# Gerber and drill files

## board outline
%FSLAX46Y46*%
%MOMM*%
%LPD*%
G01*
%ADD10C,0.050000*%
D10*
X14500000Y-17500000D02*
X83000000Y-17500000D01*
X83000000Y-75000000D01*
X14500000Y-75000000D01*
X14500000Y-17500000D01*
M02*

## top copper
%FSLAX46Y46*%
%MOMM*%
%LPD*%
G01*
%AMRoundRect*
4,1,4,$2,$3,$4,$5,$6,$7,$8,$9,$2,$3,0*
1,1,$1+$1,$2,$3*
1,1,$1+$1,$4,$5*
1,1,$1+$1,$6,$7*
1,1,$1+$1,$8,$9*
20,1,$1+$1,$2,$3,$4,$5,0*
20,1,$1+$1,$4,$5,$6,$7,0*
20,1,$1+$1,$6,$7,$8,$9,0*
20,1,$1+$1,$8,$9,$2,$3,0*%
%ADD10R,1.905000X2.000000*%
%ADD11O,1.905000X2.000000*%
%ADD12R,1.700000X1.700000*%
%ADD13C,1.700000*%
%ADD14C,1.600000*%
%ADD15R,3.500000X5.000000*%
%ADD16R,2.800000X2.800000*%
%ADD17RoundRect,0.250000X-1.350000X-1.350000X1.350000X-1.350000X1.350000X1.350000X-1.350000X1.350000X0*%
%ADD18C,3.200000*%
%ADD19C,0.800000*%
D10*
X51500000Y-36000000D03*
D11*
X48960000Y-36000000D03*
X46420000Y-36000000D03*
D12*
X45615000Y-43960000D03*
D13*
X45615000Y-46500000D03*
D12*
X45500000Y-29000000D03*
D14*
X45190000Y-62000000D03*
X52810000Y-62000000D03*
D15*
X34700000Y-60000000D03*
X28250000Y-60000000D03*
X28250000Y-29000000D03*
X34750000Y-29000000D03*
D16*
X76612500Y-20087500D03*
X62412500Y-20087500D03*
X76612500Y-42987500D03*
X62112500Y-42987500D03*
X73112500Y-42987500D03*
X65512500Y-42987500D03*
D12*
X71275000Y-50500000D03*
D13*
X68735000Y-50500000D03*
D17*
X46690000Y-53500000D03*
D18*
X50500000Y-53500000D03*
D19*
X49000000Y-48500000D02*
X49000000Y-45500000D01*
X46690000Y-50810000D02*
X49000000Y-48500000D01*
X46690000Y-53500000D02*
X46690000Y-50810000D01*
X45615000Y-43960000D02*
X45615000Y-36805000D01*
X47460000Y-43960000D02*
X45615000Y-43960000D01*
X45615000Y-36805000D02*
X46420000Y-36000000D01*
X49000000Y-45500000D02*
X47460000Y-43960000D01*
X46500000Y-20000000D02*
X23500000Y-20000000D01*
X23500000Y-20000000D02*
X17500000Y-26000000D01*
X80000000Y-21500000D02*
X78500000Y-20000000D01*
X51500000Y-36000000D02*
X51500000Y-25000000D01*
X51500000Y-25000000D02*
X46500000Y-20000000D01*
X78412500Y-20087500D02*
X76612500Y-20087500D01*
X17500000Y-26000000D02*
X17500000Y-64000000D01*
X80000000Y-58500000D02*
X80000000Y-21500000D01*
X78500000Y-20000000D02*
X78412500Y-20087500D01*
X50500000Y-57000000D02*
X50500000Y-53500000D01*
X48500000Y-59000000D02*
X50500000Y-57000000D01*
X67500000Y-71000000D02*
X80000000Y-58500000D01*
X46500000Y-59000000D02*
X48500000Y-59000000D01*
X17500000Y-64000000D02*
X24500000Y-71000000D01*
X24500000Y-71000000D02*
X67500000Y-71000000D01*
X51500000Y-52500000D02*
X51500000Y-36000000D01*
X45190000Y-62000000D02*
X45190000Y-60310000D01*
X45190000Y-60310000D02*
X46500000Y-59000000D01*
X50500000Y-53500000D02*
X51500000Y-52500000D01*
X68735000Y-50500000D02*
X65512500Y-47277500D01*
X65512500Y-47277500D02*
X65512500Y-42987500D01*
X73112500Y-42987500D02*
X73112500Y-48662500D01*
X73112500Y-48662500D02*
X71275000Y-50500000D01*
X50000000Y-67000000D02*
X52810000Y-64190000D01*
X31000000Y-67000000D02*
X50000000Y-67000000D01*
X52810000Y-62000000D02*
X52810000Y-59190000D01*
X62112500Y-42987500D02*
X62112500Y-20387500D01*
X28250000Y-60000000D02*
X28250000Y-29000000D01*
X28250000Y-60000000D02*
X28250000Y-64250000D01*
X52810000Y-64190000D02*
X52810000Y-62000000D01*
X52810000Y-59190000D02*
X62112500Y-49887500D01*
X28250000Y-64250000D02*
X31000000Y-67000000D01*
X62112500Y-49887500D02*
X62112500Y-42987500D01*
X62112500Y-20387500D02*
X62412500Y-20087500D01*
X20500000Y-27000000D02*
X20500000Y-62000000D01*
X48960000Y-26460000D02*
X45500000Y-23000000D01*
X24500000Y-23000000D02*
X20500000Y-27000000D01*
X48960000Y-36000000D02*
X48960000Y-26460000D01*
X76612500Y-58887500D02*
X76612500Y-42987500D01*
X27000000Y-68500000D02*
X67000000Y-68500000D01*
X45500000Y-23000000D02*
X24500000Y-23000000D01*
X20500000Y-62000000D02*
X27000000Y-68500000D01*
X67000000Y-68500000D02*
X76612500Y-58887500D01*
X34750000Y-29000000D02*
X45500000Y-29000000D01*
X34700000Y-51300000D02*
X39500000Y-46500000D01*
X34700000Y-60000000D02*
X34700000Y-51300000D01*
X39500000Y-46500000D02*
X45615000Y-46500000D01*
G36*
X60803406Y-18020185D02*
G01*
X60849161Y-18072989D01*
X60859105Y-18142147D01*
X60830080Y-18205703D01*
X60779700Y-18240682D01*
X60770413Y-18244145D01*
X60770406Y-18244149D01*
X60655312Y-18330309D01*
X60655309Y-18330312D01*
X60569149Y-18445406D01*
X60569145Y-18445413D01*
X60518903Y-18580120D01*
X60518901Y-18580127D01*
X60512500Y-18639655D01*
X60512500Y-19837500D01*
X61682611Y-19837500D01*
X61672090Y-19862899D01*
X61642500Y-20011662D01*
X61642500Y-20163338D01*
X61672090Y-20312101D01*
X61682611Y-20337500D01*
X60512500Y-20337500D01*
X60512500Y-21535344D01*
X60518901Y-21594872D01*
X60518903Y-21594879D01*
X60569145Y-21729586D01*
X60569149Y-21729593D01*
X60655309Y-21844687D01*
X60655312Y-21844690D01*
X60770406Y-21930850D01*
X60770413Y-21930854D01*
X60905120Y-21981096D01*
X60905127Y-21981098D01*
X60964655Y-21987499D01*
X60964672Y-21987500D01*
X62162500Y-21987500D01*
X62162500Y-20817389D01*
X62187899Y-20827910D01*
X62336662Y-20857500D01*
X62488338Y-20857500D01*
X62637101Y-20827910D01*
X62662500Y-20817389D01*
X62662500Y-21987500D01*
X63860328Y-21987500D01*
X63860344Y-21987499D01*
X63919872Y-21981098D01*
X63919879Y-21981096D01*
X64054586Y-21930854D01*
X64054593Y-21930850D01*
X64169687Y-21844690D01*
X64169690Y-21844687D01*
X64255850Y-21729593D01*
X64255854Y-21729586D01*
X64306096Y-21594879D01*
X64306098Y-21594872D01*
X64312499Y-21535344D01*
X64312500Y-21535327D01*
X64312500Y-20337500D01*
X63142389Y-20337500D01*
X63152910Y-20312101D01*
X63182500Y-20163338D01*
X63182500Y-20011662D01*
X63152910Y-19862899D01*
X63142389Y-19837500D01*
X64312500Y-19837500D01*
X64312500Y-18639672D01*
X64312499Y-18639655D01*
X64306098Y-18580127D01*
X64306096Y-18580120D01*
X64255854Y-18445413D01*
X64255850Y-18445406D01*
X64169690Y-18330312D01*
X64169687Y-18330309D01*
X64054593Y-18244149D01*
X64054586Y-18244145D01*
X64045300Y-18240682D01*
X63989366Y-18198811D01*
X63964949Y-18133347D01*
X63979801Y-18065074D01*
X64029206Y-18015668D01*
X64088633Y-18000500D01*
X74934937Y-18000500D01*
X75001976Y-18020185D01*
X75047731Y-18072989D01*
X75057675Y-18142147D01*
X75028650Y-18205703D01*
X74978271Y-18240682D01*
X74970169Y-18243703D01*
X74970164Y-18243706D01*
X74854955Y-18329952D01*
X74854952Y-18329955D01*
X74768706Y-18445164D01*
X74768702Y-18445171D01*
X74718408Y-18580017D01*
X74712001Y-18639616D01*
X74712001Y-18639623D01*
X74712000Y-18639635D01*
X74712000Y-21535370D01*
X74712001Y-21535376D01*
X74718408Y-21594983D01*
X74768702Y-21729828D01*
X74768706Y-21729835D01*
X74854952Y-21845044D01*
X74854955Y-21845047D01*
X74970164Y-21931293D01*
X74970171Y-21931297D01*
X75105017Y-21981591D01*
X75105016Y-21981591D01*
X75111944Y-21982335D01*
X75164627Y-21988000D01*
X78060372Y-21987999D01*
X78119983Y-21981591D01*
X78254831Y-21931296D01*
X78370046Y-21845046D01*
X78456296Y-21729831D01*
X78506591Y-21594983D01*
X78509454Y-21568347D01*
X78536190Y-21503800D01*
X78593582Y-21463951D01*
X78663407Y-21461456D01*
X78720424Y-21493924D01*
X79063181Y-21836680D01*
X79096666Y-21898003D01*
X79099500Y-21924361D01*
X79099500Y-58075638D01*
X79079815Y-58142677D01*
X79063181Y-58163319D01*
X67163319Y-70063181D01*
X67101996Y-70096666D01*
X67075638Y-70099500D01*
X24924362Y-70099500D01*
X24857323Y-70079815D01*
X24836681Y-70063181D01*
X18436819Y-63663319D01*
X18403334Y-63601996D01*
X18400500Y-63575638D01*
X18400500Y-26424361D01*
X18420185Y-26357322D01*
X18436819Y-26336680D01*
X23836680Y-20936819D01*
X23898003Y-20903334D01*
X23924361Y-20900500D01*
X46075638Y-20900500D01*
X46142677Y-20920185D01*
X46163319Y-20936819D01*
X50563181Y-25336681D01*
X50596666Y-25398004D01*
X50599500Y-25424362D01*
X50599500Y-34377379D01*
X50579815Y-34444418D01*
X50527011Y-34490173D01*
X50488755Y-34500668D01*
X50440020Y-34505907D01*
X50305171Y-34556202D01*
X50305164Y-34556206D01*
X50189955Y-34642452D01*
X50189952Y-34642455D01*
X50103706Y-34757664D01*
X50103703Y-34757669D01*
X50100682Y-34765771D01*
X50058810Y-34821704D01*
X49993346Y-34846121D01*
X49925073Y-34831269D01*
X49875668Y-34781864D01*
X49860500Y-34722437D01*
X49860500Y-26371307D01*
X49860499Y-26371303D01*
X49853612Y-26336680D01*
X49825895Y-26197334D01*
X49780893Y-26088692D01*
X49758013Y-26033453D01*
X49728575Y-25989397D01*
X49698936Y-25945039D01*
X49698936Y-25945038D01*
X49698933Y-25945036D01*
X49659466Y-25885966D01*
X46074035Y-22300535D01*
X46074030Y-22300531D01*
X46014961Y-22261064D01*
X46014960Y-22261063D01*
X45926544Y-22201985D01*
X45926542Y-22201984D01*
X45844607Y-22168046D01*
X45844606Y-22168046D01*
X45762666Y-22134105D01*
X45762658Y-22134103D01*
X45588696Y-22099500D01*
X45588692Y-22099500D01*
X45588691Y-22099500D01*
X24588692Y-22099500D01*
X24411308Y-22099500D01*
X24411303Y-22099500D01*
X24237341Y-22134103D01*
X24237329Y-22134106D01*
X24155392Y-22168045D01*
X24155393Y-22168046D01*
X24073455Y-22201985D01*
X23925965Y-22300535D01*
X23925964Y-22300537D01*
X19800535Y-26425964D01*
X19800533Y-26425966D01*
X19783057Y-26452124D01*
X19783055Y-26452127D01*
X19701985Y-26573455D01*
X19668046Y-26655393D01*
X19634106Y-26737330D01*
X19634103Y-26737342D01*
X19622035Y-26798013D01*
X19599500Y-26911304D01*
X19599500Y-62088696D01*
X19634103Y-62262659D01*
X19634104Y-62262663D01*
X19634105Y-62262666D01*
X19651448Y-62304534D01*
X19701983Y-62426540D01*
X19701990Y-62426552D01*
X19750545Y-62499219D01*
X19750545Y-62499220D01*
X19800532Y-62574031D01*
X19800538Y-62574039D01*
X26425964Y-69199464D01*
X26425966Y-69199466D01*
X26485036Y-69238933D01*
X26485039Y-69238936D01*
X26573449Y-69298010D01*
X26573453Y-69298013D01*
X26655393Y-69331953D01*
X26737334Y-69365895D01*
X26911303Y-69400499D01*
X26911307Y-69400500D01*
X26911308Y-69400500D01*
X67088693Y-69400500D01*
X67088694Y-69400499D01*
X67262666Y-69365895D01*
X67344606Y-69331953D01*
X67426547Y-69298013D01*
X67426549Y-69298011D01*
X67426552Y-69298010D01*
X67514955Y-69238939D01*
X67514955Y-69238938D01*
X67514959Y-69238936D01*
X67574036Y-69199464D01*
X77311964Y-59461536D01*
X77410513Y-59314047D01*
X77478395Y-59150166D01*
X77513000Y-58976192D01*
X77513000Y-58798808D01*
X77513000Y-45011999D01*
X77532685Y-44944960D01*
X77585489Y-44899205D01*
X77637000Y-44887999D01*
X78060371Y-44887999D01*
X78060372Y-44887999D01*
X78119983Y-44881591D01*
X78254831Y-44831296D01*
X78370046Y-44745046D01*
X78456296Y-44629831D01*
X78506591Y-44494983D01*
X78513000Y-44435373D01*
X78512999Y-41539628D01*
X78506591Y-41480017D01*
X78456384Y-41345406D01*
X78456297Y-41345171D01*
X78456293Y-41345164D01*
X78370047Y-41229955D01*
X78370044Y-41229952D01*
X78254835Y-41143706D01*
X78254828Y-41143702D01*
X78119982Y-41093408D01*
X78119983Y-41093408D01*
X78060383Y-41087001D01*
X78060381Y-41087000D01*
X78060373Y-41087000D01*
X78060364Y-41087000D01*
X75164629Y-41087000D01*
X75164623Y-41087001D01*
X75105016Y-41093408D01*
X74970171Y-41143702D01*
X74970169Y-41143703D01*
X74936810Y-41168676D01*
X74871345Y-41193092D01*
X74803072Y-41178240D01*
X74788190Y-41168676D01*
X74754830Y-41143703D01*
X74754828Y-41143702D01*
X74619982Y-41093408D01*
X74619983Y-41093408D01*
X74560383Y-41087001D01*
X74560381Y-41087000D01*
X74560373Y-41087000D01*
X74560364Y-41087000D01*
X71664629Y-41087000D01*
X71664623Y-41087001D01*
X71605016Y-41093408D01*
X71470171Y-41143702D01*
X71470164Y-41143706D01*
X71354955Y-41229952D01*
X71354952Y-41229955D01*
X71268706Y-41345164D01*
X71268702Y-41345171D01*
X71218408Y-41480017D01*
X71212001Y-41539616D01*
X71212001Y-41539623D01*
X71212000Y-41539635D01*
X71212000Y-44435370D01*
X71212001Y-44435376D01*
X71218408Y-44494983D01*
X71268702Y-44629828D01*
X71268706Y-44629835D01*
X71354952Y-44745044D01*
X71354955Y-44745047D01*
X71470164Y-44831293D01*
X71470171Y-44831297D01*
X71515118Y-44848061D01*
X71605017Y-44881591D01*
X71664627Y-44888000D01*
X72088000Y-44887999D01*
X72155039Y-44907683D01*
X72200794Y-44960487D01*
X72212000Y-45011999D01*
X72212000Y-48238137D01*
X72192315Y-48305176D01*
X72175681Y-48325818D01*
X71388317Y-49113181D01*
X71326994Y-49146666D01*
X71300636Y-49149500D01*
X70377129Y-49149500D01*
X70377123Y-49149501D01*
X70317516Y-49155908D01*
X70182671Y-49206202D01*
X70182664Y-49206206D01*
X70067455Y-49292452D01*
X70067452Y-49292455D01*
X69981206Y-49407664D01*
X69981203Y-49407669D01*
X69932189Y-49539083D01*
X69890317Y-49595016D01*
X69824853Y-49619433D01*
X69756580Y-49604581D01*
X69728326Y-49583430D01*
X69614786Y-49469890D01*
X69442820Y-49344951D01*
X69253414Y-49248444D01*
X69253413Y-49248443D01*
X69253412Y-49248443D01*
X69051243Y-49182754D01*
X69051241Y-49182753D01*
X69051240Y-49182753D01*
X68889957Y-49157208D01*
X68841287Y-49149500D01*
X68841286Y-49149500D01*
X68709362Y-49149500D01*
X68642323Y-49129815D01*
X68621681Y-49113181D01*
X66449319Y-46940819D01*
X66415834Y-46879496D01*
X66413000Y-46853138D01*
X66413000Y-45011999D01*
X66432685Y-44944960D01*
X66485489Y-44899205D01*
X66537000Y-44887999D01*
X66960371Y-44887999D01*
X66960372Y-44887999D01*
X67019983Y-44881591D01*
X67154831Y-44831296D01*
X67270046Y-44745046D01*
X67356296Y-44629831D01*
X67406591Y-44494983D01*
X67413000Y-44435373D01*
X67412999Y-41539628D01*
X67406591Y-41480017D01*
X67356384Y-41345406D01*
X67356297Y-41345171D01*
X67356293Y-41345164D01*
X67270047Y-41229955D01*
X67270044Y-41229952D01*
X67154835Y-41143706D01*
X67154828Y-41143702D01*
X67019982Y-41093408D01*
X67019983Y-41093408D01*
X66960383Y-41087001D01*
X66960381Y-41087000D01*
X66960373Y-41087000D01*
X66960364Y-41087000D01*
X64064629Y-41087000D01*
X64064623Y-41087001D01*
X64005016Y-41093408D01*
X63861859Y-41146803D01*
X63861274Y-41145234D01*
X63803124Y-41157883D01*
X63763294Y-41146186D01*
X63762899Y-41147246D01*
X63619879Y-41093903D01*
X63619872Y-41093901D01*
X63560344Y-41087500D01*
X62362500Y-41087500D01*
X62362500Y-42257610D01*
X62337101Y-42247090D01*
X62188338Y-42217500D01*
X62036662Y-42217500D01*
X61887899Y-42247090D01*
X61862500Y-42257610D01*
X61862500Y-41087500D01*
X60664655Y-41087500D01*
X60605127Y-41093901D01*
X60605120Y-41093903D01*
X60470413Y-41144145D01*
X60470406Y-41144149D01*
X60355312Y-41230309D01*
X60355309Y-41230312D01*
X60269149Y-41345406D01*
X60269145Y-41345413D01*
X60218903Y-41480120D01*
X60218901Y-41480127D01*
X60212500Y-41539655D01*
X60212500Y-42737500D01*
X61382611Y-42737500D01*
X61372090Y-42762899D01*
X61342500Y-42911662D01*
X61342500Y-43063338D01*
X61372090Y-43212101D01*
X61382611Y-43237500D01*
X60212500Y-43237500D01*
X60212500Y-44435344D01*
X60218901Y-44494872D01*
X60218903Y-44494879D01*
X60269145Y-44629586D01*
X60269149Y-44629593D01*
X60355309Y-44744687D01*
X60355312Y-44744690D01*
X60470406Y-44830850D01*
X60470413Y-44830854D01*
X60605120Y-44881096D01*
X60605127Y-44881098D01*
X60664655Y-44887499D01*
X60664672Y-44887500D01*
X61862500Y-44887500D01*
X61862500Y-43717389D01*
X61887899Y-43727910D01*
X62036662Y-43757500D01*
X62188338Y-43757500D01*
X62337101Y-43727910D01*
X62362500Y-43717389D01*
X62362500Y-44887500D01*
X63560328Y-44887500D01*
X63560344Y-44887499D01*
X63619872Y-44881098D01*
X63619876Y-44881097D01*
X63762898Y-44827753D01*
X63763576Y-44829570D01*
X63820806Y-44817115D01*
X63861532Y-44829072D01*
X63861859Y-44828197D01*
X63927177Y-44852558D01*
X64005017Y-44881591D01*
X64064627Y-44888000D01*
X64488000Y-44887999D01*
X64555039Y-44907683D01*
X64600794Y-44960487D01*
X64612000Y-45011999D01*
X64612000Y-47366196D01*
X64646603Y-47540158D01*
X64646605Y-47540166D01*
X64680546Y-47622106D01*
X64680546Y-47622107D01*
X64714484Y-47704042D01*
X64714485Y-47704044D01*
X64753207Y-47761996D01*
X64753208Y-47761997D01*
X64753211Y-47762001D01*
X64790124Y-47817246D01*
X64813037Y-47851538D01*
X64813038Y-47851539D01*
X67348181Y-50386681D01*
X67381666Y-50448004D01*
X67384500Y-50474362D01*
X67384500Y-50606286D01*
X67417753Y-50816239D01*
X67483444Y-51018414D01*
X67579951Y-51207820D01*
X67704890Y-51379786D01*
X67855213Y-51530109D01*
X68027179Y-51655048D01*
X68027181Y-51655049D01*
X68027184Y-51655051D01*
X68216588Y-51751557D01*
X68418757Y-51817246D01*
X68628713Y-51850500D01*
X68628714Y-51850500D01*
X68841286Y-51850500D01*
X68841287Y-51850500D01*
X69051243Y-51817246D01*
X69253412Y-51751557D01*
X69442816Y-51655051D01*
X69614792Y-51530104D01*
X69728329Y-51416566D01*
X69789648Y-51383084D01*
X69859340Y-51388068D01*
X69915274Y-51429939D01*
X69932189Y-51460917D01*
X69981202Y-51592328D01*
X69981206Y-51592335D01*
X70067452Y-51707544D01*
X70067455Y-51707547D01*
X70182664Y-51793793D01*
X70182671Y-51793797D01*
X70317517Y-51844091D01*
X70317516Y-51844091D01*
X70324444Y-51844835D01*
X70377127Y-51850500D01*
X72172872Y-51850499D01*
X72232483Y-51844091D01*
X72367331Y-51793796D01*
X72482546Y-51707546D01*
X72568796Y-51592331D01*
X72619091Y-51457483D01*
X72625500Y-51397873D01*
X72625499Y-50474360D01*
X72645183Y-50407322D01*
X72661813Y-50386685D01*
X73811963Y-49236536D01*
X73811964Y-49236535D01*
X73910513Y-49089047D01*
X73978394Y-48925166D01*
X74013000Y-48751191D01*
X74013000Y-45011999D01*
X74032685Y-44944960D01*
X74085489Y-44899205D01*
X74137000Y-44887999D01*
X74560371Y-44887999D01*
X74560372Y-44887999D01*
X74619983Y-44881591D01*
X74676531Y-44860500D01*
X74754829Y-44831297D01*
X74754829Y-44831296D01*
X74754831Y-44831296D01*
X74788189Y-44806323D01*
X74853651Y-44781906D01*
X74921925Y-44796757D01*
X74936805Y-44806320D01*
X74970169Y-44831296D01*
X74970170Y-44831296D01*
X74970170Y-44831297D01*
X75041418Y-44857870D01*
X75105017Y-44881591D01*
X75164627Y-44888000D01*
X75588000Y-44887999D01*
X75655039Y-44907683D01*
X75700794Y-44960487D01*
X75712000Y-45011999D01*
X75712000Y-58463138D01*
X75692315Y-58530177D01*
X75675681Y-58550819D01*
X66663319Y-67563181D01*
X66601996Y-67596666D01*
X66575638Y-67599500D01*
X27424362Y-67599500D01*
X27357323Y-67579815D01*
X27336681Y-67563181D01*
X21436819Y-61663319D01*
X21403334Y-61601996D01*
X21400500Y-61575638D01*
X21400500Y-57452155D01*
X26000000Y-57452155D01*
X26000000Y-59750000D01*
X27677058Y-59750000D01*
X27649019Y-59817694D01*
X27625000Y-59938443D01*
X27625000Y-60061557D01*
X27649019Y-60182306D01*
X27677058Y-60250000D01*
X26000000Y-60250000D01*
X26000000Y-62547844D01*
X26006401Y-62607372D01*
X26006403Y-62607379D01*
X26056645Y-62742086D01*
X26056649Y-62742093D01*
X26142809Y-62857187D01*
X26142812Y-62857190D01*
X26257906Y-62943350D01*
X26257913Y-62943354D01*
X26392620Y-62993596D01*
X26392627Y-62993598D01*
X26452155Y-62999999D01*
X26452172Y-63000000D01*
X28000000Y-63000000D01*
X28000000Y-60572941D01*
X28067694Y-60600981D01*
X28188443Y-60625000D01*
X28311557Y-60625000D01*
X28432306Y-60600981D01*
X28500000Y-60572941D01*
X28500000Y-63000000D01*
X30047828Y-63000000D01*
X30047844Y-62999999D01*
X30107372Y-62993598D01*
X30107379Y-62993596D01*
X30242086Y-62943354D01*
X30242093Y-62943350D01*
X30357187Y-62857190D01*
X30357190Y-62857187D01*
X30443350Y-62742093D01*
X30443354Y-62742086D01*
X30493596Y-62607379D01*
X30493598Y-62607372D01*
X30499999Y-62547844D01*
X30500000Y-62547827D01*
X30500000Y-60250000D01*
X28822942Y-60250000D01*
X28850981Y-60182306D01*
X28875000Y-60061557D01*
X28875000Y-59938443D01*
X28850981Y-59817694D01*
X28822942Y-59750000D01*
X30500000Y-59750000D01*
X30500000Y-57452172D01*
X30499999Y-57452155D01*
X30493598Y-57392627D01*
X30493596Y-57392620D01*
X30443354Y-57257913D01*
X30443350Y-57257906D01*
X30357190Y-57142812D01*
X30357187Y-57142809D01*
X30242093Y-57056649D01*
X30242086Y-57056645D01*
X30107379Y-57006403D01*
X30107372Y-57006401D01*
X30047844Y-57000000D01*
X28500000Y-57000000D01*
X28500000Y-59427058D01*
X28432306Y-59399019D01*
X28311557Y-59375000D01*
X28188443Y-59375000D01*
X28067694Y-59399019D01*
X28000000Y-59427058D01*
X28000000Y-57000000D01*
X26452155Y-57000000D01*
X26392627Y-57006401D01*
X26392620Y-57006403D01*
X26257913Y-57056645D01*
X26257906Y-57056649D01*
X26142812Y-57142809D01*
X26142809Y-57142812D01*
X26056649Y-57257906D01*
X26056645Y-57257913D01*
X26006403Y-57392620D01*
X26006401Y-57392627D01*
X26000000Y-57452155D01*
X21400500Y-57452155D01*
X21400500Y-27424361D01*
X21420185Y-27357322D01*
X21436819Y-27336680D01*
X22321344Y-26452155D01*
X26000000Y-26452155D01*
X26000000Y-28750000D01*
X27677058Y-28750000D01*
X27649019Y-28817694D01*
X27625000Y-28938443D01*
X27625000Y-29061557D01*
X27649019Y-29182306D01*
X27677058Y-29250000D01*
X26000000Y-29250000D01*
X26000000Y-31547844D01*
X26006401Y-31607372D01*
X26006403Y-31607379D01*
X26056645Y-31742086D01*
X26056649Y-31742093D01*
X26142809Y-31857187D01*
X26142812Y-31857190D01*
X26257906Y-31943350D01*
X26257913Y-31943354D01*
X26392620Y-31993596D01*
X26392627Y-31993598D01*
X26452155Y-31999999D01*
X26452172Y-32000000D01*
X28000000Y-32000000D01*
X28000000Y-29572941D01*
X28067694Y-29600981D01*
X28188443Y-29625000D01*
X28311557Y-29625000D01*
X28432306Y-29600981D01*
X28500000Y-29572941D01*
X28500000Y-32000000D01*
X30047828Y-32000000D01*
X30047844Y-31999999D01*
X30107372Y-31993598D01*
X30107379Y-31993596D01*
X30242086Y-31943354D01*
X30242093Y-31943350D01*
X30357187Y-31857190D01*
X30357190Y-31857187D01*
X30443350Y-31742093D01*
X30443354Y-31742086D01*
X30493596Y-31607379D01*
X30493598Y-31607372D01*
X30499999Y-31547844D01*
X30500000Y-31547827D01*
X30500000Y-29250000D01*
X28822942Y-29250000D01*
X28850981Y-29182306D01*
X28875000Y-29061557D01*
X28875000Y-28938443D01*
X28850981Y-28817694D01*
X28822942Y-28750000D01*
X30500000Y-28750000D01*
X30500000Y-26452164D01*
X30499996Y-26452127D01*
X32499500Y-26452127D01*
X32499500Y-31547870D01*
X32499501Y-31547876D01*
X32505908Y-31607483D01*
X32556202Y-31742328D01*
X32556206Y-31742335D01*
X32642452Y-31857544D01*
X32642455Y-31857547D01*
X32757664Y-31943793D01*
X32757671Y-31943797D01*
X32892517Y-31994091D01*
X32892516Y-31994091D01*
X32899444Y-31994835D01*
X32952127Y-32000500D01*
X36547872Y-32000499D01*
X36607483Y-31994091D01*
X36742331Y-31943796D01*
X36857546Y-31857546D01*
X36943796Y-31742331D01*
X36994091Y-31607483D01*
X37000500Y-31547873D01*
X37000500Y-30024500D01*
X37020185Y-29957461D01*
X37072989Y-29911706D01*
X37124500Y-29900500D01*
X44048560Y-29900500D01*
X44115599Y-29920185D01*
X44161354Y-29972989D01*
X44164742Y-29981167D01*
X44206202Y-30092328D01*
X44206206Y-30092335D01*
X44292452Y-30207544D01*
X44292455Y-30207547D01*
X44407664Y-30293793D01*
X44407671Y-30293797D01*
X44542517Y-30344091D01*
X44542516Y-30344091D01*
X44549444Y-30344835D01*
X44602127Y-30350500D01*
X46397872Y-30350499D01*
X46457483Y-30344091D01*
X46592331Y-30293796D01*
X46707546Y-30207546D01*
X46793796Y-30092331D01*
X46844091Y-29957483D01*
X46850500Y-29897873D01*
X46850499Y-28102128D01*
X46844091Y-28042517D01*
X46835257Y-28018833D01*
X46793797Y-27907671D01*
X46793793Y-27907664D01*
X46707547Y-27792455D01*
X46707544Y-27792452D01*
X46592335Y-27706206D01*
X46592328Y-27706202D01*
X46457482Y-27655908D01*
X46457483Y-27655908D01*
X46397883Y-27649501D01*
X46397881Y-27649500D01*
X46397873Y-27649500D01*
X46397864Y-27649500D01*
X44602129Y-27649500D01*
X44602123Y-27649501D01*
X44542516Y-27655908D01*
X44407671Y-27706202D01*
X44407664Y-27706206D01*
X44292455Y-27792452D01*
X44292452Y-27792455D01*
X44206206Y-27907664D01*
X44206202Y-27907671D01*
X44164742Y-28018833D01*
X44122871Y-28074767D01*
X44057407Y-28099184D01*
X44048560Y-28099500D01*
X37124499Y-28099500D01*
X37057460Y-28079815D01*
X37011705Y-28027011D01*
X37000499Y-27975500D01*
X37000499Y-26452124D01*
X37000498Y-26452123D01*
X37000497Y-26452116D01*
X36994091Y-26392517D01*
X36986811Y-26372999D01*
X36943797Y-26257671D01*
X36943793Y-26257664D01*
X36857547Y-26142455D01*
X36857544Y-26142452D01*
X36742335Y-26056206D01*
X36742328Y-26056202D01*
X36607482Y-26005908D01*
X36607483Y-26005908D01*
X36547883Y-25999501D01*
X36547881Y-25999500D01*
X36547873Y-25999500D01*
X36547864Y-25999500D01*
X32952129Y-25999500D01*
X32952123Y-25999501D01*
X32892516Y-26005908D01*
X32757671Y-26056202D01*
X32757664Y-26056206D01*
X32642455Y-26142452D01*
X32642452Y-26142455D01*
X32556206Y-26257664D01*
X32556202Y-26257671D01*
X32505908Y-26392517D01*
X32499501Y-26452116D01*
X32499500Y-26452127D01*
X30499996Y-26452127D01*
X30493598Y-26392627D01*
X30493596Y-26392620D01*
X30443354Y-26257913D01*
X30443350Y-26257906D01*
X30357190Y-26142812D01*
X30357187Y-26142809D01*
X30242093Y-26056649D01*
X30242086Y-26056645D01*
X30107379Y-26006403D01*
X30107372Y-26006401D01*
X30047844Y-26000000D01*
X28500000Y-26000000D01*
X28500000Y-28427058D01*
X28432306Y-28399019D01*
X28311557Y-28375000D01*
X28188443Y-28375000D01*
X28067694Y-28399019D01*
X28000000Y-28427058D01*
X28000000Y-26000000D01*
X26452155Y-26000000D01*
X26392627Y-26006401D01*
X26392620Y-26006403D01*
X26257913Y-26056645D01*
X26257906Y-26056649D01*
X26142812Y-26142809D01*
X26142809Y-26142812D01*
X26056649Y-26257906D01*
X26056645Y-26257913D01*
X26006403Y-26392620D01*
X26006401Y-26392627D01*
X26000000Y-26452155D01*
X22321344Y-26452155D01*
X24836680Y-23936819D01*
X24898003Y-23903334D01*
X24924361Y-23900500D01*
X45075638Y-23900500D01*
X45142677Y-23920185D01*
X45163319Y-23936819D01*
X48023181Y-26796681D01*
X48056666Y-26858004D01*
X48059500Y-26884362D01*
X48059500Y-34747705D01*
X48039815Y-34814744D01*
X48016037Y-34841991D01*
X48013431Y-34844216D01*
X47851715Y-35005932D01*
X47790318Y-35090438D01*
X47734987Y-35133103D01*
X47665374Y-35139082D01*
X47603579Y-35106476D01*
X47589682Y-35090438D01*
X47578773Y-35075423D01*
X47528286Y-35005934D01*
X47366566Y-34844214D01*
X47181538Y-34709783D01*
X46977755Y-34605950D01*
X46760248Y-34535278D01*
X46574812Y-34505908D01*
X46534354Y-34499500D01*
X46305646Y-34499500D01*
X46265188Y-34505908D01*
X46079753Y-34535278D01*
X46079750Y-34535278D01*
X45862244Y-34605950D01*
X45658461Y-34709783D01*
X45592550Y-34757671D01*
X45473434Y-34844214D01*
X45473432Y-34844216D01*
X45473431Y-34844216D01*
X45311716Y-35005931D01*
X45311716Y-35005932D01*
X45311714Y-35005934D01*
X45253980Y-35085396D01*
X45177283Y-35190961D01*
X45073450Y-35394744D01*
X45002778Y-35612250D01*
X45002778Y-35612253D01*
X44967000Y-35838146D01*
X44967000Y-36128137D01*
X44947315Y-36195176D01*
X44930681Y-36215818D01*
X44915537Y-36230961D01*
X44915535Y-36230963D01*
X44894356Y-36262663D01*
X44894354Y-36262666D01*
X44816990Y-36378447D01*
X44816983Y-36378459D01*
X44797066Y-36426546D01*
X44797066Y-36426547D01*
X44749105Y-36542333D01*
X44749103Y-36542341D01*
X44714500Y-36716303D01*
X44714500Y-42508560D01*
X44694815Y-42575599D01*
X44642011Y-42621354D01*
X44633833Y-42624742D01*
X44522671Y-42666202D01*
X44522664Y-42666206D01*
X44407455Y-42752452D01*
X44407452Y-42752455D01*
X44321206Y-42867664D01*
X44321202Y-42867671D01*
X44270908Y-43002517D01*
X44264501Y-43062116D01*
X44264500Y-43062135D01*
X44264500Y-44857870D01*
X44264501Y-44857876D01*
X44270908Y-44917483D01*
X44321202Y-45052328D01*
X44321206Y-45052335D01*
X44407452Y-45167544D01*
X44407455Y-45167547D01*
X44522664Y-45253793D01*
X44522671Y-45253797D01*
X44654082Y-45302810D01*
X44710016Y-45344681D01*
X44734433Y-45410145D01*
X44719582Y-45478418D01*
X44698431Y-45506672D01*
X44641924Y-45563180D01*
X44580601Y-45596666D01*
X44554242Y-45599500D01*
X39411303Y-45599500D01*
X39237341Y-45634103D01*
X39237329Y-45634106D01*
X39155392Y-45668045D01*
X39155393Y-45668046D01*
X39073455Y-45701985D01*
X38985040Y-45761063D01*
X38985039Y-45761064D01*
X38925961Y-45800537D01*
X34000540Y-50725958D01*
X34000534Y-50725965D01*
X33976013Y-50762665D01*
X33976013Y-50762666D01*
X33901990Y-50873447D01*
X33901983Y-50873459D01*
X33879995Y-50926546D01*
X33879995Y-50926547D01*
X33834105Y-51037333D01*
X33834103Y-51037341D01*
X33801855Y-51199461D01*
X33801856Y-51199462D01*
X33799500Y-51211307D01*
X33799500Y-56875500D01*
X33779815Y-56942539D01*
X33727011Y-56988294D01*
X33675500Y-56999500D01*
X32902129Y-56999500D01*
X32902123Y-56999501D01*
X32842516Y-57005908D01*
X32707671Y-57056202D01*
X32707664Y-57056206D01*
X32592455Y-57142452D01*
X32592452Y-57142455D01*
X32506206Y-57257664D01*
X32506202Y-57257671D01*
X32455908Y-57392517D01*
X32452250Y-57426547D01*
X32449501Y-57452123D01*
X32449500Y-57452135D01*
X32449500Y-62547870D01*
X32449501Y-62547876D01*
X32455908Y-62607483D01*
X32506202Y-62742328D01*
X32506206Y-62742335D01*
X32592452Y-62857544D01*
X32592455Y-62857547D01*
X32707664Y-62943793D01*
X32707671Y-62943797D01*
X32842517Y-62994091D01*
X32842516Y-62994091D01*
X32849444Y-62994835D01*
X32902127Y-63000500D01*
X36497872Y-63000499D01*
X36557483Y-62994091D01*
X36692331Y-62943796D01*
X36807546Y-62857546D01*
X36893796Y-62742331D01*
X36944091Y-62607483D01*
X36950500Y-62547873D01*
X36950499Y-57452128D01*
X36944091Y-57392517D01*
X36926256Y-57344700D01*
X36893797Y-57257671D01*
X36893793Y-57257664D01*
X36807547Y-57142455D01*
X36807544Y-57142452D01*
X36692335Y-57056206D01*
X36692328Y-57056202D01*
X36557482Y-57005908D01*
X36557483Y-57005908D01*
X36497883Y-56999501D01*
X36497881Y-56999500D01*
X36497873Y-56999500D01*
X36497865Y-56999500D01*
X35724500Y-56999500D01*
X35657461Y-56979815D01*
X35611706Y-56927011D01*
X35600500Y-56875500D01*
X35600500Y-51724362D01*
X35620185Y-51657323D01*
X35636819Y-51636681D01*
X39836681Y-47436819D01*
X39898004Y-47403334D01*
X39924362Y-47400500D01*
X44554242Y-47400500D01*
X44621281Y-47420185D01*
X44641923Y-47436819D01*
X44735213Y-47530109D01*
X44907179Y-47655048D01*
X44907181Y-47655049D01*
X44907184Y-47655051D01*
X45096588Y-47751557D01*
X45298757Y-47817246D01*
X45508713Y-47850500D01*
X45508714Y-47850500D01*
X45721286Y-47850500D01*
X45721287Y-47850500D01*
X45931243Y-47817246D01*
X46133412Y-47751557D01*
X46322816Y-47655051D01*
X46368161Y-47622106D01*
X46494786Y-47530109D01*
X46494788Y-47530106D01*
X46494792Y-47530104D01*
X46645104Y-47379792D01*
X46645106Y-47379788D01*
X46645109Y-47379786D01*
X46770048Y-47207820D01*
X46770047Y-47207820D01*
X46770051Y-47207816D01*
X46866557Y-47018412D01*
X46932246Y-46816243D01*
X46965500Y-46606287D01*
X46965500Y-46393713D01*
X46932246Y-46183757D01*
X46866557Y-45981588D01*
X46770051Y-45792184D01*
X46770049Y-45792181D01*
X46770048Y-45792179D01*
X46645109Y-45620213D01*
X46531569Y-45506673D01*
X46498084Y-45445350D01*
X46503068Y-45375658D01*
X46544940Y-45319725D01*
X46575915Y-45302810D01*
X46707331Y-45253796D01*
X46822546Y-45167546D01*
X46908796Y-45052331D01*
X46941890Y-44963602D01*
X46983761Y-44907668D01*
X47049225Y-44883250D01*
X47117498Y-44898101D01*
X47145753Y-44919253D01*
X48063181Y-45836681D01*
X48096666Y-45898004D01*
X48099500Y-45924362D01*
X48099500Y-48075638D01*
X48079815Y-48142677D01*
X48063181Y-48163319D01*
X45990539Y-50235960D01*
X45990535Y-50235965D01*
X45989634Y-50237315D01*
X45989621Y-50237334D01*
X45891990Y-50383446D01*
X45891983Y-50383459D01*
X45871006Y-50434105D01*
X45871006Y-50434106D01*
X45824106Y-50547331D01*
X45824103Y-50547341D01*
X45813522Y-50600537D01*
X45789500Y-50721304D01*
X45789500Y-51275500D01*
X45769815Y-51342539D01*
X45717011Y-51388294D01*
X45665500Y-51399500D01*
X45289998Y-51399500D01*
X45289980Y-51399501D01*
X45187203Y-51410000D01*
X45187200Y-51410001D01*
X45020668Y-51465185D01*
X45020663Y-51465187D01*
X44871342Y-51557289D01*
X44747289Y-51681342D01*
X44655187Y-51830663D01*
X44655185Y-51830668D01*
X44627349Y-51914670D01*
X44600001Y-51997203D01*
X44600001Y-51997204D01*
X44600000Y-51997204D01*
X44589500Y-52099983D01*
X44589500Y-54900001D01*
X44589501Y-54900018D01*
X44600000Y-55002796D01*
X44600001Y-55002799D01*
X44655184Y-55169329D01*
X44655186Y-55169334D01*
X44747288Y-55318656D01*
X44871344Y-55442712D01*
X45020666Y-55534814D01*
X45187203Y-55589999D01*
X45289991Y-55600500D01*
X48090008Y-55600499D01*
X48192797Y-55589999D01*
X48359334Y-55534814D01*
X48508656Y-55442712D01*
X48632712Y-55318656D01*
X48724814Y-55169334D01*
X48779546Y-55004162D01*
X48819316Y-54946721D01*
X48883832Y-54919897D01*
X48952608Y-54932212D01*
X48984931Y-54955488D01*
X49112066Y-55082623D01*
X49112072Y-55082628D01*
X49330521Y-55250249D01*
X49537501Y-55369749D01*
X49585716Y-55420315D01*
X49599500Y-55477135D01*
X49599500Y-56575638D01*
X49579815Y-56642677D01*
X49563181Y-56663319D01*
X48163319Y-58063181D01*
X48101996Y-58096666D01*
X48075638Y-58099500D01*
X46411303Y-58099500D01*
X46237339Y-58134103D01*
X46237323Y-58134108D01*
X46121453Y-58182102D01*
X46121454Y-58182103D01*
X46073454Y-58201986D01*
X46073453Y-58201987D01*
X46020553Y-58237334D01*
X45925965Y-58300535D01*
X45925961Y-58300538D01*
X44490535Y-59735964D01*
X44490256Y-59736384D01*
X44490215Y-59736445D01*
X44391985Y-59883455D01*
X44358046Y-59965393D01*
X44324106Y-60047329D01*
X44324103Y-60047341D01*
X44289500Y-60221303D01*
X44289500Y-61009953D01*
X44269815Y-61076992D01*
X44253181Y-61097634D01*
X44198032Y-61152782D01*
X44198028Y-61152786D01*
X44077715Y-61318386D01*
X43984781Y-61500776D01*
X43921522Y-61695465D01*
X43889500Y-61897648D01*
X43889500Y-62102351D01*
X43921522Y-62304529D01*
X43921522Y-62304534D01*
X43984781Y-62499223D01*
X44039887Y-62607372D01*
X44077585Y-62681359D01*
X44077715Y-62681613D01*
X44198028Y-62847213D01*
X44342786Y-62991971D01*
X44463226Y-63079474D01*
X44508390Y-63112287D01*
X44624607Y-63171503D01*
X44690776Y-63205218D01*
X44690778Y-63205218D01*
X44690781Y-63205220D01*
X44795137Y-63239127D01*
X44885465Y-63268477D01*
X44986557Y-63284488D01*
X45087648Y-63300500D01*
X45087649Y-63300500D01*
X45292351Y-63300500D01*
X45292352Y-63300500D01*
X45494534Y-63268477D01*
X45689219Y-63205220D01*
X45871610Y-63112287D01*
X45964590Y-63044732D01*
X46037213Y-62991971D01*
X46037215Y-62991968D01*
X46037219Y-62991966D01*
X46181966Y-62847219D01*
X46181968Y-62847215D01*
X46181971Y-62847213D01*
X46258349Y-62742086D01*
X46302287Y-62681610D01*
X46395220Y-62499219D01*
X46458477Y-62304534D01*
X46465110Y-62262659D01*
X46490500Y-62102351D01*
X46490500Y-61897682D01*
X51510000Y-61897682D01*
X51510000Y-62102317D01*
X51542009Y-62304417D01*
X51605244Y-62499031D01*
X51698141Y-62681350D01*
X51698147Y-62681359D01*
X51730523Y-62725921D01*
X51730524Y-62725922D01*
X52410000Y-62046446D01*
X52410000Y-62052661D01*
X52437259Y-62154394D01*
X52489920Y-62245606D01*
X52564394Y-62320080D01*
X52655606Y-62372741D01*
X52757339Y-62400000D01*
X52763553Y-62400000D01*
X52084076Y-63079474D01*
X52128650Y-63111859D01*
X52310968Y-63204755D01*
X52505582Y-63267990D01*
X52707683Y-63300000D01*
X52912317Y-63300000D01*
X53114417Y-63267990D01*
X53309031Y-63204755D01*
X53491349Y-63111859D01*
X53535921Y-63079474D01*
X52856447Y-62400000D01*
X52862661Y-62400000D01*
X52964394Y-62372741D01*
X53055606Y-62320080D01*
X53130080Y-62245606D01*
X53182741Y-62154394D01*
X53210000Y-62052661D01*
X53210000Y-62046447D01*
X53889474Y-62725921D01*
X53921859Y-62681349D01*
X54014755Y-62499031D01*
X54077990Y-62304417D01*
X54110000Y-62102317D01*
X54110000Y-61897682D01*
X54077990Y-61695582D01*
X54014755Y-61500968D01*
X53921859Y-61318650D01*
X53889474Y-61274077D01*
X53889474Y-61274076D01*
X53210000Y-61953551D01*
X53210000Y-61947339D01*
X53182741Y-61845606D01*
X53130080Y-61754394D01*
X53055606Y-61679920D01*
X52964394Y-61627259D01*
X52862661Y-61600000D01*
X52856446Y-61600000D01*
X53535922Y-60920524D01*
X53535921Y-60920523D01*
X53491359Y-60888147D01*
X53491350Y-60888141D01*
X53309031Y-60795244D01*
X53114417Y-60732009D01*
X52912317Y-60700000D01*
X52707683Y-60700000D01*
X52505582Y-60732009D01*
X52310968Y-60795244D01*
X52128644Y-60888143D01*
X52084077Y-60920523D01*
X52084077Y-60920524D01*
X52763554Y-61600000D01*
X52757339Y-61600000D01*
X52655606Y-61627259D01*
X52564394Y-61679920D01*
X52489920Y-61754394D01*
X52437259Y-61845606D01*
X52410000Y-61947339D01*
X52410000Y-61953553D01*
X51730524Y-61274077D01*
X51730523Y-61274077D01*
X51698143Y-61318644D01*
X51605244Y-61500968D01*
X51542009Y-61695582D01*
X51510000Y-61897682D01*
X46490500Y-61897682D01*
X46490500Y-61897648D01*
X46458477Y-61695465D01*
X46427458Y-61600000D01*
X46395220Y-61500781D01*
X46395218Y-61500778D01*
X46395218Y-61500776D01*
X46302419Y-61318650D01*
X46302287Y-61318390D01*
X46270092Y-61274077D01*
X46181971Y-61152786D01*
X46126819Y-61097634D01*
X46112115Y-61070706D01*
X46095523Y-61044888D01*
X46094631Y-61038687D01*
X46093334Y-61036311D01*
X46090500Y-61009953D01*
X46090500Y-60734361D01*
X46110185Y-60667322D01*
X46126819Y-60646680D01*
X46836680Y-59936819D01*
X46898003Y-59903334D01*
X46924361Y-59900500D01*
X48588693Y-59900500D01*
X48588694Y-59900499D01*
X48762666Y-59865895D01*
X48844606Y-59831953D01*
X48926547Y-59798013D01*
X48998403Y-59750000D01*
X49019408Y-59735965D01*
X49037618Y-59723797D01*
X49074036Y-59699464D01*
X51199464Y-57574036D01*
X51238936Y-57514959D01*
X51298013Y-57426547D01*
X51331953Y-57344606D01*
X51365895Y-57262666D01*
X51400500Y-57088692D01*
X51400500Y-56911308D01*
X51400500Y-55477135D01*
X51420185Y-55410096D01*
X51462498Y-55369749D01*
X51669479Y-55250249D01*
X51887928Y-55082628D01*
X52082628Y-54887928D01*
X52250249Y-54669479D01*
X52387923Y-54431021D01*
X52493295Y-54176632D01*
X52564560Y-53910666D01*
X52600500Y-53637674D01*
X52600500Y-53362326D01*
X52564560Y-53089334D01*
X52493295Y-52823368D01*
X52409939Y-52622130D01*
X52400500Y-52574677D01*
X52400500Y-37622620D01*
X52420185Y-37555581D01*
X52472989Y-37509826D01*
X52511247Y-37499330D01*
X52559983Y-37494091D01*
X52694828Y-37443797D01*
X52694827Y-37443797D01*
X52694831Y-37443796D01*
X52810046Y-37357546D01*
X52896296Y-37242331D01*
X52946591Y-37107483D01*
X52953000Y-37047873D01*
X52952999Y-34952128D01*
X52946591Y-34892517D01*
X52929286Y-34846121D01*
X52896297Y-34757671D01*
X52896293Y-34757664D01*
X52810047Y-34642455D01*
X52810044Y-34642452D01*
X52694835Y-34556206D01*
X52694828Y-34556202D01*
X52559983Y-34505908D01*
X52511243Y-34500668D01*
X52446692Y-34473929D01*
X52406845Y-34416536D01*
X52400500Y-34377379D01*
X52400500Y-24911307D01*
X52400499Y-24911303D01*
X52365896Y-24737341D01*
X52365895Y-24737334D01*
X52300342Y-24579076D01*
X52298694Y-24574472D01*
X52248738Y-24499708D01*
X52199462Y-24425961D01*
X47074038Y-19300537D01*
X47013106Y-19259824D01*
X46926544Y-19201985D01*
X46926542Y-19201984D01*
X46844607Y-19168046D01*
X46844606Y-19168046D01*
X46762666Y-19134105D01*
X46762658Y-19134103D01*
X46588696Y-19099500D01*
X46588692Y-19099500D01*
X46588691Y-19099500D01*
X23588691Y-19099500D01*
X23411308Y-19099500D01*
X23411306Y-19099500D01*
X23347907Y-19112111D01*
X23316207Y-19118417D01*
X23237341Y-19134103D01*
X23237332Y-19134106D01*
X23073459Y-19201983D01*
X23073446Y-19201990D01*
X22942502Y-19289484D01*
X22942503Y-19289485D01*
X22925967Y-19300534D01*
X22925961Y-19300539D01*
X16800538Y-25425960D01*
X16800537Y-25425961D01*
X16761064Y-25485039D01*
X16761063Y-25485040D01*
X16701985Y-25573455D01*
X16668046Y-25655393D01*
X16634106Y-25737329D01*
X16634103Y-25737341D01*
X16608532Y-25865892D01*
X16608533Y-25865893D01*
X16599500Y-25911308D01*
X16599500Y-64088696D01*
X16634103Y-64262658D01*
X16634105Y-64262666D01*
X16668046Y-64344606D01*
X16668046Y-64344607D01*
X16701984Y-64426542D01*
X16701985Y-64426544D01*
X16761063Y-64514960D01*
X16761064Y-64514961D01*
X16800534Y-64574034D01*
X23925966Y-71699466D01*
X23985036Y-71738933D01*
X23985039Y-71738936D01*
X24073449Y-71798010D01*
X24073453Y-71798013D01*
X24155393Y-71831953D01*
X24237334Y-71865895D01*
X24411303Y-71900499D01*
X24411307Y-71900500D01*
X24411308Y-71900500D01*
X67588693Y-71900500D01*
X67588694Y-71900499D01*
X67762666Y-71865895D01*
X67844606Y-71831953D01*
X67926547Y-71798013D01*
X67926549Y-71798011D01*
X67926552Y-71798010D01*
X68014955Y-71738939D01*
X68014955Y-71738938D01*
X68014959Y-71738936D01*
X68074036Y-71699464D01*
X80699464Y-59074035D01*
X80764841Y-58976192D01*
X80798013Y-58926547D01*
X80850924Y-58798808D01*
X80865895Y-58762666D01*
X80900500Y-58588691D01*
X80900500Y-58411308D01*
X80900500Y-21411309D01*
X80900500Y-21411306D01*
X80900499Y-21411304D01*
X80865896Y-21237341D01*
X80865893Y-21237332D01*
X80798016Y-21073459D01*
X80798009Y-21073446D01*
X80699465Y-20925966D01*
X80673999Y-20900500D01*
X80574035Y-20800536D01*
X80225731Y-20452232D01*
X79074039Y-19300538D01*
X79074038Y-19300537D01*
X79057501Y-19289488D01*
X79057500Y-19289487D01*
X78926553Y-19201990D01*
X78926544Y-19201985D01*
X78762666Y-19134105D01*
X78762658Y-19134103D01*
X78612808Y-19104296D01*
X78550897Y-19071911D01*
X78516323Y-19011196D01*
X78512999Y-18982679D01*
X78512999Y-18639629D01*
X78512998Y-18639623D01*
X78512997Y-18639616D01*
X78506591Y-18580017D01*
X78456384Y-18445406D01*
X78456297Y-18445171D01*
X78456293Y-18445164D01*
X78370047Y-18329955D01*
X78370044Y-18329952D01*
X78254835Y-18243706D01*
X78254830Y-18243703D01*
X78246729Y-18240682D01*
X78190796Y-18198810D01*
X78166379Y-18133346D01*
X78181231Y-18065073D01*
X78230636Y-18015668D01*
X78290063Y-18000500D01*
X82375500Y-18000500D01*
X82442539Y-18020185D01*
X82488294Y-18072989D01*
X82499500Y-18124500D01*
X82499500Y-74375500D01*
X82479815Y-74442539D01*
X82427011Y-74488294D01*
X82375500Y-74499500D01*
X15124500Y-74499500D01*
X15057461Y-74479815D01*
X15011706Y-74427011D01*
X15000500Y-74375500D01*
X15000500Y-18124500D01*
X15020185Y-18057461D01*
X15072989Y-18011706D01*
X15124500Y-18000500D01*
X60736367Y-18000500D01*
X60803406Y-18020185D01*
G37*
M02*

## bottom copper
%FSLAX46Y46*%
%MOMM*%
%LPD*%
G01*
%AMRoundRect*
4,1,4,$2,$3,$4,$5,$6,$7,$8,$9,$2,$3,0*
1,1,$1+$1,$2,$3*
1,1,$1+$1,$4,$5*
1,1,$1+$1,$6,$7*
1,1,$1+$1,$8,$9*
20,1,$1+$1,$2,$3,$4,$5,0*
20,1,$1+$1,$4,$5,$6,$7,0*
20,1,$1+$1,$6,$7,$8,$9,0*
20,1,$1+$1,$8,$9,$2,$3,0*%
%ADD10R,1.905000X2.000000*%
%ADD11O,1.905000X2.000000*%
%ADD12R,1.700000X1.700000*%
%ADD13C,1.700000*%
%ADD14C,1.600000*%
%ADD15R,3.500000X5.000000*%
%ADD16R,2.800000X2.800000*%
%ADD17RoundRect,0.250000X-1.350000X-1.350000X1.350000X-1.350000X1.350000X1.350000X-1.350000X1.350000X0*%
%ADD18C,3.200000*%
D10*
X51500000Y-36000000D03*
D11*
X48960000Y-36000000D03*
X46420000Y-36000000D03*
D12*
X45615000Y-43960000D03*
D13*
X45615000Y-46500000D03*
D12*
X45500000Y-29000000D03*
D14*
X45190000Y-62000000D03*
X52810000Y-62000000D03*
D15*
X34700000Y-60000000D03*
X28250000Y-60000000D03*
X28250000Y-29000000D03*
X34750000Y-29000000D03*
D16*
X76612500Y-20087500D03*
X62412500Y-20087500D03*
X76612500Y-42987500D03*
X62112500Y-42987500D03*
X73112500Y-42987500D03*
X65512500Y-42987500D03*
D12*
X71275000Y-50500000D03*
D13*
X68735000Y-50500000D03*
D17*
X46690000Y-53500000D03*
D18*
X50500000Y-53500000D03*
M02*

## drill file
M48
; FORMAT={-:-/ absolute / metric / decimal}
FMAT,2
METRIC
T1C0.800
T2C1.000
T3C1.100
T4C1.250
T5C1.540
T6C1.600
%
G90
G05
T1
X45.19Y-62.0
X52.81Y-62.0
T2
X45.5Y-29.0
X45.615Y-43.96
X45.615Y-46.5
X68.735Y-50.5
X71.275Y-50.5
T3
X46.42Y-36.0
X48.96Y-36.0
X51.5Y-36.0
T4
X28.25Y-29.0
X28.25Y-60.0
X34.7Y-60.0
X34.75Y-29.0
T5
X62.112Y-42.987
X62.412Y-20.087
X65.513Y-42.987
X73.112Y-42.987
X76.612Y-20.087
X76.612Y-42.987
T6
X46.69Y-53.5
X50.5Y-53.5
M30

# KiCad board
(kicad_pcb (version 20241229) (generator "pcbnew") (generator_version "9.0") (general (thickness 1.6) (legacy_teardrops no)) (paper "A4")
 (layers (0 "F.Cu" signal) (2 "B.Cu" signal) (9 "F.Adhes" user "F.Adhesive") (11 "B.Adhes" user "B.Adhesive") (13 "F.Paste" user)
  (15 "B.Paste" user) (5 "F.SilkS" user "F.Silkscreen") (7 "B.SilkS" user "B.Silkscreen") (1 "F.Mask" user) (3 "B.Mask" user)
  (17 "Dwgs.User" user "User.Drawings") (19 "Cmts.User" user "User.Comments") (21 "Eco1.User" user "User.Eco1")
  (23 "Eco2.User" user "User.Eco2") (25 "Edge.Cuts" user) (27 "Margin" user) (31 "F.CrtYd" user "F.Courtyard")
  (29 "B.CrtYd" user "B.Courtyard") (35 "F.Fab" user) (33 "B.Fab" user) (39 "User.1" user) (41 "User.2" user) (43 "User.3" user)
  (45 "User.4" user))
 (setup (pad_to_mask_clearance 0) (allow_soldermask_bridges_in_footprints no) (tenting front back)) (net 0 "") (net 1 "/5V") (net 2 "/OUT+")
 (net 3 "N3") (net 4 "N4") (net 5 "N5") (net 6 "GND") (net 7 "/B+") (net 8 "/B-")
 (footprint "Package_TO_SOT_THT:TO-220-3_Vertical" (layer "F.Cu") (at 51.5 36 180)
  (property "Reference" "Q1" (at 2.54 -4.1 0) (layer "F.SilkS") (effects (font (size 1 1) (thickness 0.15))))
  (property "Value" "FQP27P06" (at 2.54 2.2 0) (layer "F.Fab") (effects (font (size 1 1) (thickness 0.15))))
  (pad "1" thru_hole rect (at 0 0 180) (size 1.905 2) (drill 1.1) (layers "*.Cu" "*.Mask") (remove_unused_layers no) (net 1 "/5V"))
  (pad "2" thru_hole oval (at 2.54 0 180) (size 1.905 2) (drill 1.1) (layers "*.Cu" "*.Mask") (remove_unused_layers no) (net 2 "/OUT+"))
  (pad "3" thru_hole oval (at 5.08 0 180) (size 1.905 2) (drill 1.1) (layers "*.Cu" "*.Mask") (remove_unused_layers no) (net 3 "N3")))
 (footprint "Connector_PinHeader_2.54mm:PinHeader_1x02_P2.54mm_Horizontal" (layer "F.Cu") (at 45.615 43.96)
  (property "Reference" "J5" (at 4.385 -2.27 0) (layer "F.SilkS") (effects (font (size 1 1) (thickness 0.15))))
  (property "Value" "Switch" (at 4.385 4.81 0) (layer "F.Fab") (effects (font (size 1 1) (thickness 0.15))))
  (pad "1" thru_hole rect (at 0 0) (size 1.7 1.7) (drill 1) (layers "*.Cu" "*.Mask") (remove_unused_layers no) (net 3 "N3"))
  (pad "2" thru_hole circle (at 0 2.54) (size 1.7 1.7) (drill 1) (layers "*.Cu" "*.Mask") (remove_unused_layers no) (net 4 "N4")))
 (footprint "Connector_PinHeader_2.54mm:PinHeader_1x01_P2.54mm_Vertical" (layer "F.Cu") (at 45.5 29)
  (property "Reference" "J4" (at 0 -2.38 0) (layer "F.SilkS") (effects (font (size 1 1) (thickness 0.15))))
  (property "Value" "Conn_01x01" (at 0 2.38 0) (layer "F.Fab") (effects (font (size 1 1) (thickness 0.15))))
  (pad "1" thru_hole rect (at 0 0) (size 1.7 1.7) (drill 1) (layers "*.Cu" "*.Mask") (remove_unused_layers no) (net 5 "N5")))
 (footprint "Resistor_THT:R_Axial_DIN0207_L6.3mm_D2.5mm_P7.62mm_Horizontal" (layer "F.Cu") (at 45.19 62)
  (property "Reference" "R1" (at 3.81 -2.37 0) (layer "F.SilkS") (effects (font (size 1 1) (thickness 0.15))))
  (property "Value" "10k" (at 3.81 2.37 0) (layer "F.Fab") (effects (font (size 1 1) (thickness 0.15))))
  (pad "1" thru_hole circle (at 0 0) (size 1.6 1.6) (drill 0.8) (layers "*.Cu" "*.Mask") (remove_unused_layers no) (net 1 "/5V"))
  (pad "2" thru_hole circle (at 7.62 0) (size 1.6 1.6) (drill 0.8) (layers "*.Cu" "*.Mask") (remove_unused_layers no) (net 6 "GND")))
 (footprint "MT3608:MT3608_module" (layer "F.Cu") (at 31.5 46 -90)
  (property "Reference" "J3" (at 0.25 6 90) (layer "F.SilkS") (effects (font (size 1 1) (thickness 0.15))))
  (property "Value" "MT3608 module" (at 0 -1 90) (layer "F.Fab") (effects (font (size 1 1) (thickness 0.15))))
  (pad "1" thru_hole rect (at 14 -3.2 90) (size 5 3.5) (drill 1.25) (layers "*.Cu" "*.Mask" "F.SilkS") (remove_unused_layers no)
   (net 4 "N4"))
  (pad "2" thru_hole rect (at 14 3.25 90) (size 5 3.5) (drill 1.25) (layers "*.Cu" "*.Mask" "F.SilkS") (remove_unused_layers no)
   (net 6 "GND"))
  (pad "3" thru_hole rect (at -17 3.25 90) (size 5 3.5) (drill 1.25) (layers "*.Cu" "*.Mask" "F.SilkS") (remove_unused_layers no)
   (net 6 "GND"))
  (pad "4" thru_hole rect (at -17 -3.25 90) (size 5 3.5) (drill 1.25) (layers "*.Cu" "*.Mask" "F.SilkS") (remove_unused_layers no)
   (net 5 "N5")))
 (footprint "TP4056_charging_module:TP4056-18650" (layer "F.Cu") (at 78.3125 18.3875 -90)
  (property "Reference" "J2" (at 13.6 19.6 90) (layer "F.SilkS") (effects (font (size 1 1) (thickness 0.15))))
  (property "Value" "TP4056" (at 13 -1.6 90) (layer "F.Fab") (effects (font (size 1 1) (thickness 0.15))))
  (pad "1" thru_hole rect (at 1.7 1.7 270) (size 2.8 2.8) (drill 1.54) (layers "*.Cu" "*.Mask") (remove_unused_layers no) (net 1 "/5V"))
  (pad "2" thru_hole rect (at 1.7 15.9 270) (size 2.8 2.8) (drill 1.54) (layers "*.Cu" "*.Mask") (remove_unused_layers no) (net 6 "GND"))
  (pad "3" thru_hole rect (at 24.6 1.7 270) (size 2.8 2.8) (drill 1.54) (layers "*.Cu" "*.Mask") (remove_unused_layers no) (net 2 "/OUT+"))
  (pad "4" thru_hole rect (at 24.6 16.2 270) (size 2.8 2.8) (drill 1.54) (layers "*.Cu" "*.Mask") (remove_unused_layers no) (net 6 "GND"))
  (pad "5" thru_hole rect (at 24.6 5.2 270) (size 2.8 2.8) (drill 1.54) (layers "*.Cu" "*.Mask") (remove_unused_layers no) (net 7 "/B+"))
  (pad "6" thru_hole rect (at 24.6 12.8 270) (size 2.8 2.8) (drill 1.54) (layers "*.Cu" "*.Mask") (remove_unused_layers no) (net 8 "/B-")))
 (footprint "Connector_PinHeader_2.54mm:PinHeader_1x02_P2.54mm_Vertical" (layer "F.Cu") (at 71.275 50.5 -90)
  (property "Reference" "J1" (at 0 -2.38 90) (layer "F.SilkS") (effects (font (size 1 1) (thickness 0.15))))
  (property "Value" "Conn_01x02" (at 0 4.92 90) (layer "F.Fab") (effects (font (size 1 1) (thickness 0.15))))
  (pad "1" thru_hole rect (at 0 0 270) (size 1.7 1.7) (drill 1) (layers "*.Cu" "*.Mask") (remove_unused_layers no) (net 7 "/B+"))
  (pad "2" thru_hole circle (at 0 2.54 270) (size 1.7 1.7) (drill 1) (layers "*.Cu" "*.Mask") (remove_unused_layers no) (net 8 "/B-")))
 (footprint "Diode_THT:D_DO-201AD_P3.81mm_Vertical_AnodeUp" (layer "F.Cu") (at 46.69 53.5)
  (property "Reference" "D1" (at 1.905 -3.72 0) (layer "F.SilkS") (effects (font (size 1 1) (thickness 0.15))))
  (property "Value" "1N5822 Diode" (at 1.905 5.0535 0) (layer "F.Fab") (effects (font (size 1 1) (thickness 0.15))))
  (pad "1" thru_hole roundrect (at 0 0) (size 3.2 3.2) (drill 1.6) (layers "*.Cu" "*.Mask") (remove_unused_layers no)
   (roundrect_rratio 0.078125) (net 3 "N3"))
  (pad "2" thru_hole circle (at 3.81 0) (size 3.2 3.2) (drill 1.6) (layers "*.Cu" "*.Mask") (remove_unused_layers no) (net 1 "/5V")))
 (gr_rect (start 14.5 17.5) (end 83 75) (stroke (width 0.05) (type default)) (fill no) (layer "Edge.Cuts"))
 (segment (start 49 48.5) (end 49 45.5) (width 0.8) (layer "F.Cu") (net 3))
 (segment (start 46.69 50.81) (end 49 48.5) (width 0.8) (layer "F.Cu") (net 3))
 (segment (start 46.69 53.5) (end 46.69 50.81) (width 0.8) (layer "F.Cu") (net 3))
 (segment (start 45.615 43.96) (end 45.615 36.805) (width 0.8) (layer "F.Cu") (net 3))
 (segment (start 47.46 43.96) (end 45.615 43.96) (width 0.8) (layer "F.Cu") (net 3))
 (segment (start 45.615 36.805) (end 46.42 36) (width 0.8) (layer "F.Cu") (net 3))
 (segment (start 49 45.5) (end 47.46 43.96) (width 0.8) (layer "F.Cu") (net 3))
 (segment (start 46.5 20) (end 23.5 20) (width 0.8) (layer "F.Cu") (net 1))
 (segment (start 23.5 20) (end 17.5 26) (width 0.8) (layer "F.Cu") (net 1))
 (segment (start 80 21.5) (end 78.5 20) (width 0.8) (layer "F.Cu") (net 1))
 (segment (start 51.5 36) (end 51.5 25) (width 0.8) (layer "F.Cu") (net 1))
 (segment (start 51.5 25) (end 46.5 20) (width 0.8) (layer "F.Cu") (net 1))
 (segment (start 78.4125 20.0875) (end 76.6125 20.0875) (width 0.8) (layer "F.Cu") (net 1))
 (segment (start 17.5 26) (end 17.5 64) (width 0.8) (layer "F.Cu") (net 1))
 (segment (start 80 58.5) (end 80 21.5) (width 0.8) (layer "F.Cu") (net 1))
 (segment (start 78.5 20) (end 78.4125 20.0875) (width 0.8) (layer "F.Cu") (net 1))
 (segment (start 50.5 57) (end 50.5 53.5) (width 0.8) (layer "F.Cu") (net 1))
 (segment (start 48.5 59) (end 50.5 57) (width 0.8) (layer "F.Cu") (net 1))
 (segment (start 67.5 71) (end 80 58.5) (width 0.8) (layer "F.Cu") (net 1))
 (segment (start 46.5 59) (end 48.5 59) (width 0.8) (layer "F.Cu") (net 1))
 (segment (start 17.5 64) (end 24.5 71) (width 0.8) (layer "F.Cu") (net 1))
 (segment (start 24.5 71) (end 67.5 71) (width 0.8) (layer "F.Cu") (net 1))
 (segment (start 51.5 52.5) (end 51.5 36) (width 0.8) (layer "F.Cu") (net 1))
 (segment (start 45.19 62) (end 45.19 60.31) (width 0.8) (layer "F.Cu") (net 1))
 (segment (start 45.19 60.31) (end 46.5 59) (width 0.8) (layer "F.Cu") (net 1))
 (segment (start 50.5 53.5) (end 51.5 52.5) (width 0.8) (layer "F.Cu") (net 1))
 (segment (start 68.735 50.5) (end 65.5125 47.2775) (width 0.8) (layer "F.Cu") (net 8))
 (segment (start 65.5125 47.2775) (end 65.5125 42.9875) (width 0.8) (layer "F.Cu") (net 8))
 (segment (start 73.1125 42.9875) (end 73.1125 48.6625) (width 0.8) (layer "F.Cu") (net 7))
 (segment (start 73.1125 48.6625) (end 71.275 50.5) (width 0.8) (layer "F.Cu") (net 7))
 (segment (start 50 67) (end 52.81 64.19) (width 0.8) (layer "F.Cu") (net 6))
 (segment (start 31 67) (end 50 67) (width 0.8) (layer "F.Cu") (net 6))
 (segment (start 52.81 62) (end 52.81 59.19) (width 0.8) (layer "F.Cu") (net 6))
 (segment (start 62.1125 42.9875) (end 62.1125 20.3875) (width 0.8) (layer "F.Cu") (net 6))
 (segment (start 28.25 60) (end 28.25 29) (width 0.8) (layer "F.Cu") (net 6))
 (segment (start 28.25 60) (end 28.25 64.25) (width 0.8) (layer "F.Cu") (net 6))
 (segment (start 52.81 64.19) (end 52.81 62) (width 0.8) (layer "F.Cu") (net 6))
 (segment (start 52.81 59.19) (end 62.1125 49.8875) (width 0.8) (layer "F.Cu") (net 6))
 (segment (start 28.25 64.25) (end 31 67) (width 0.8) (layer "F.Cu") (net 6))
 (segment (start 62.1125 49.8875) (end 62.1125 42.9875) (width 0.8) (layer "F.Cu") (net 6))
 (segment (start 62.1125 20.3875) (end 62.4125 20.0875) (width 0.8) (layer "F.Cu") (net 6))
 (segment (start 20.5 27) (end 20.5 62) (width 0.8) (layer "F.Cu") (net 2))
 (segment (start 48.96 26.46) (end 45.5 23) (width 0.8) (layer "F.Cu") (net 2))
 (segment (start 24.5 23) (end 20.5 27) (width 0.8) (layer "F.Cu") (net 2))
 (segment (start 48.96 36) (end 48.96 26.46) (width 0.8) (layer "F.Cu") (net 2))
 (segment (start 76.6125 58.8875) (end 76.6125 42.9875) (width 0.8) (layer "F.Cu") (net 2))
 (segment (start 27 68.5) (end 67 68.5) (width 0.8) (layer "F.Cu") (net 2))
 (segment (start 45.5 23) (end 24.5 23) (width 0.8) (layer "F.Cu") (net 2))
 (segment (start 20.5 62) (end 27 68.5) (width 0.8) (layer "F.Cu") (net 2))
 (segment (start 67 68.5) (end 76.6125 58.8875) (width 0.8) (layer "F.Cu") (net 2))
 (segment (start 34.75 29) (end 45.5 29) (width 0.8) (layer "F.Cu") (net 5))
 (segment (start 34.7 51.3) (end 39.5 46.5) (width 0.8) (layer "F.Cu") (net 4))
 (segment (start 34.7 60) (end 34.7 51.3) (width 0.8) (layer "F.Cu") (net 4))
 (segment (start 39.5 46.5) (end 45.615 46.5) (width 0.8) (layer "F.Cu") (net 4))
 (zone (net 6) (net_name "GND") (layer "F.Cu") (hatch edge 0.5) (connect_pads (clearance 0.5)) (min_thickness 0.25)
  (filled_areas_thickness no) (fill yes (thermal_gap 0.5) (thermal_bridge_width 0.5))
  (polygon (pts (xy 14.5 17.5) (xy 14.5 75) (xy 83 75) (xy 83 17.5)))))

